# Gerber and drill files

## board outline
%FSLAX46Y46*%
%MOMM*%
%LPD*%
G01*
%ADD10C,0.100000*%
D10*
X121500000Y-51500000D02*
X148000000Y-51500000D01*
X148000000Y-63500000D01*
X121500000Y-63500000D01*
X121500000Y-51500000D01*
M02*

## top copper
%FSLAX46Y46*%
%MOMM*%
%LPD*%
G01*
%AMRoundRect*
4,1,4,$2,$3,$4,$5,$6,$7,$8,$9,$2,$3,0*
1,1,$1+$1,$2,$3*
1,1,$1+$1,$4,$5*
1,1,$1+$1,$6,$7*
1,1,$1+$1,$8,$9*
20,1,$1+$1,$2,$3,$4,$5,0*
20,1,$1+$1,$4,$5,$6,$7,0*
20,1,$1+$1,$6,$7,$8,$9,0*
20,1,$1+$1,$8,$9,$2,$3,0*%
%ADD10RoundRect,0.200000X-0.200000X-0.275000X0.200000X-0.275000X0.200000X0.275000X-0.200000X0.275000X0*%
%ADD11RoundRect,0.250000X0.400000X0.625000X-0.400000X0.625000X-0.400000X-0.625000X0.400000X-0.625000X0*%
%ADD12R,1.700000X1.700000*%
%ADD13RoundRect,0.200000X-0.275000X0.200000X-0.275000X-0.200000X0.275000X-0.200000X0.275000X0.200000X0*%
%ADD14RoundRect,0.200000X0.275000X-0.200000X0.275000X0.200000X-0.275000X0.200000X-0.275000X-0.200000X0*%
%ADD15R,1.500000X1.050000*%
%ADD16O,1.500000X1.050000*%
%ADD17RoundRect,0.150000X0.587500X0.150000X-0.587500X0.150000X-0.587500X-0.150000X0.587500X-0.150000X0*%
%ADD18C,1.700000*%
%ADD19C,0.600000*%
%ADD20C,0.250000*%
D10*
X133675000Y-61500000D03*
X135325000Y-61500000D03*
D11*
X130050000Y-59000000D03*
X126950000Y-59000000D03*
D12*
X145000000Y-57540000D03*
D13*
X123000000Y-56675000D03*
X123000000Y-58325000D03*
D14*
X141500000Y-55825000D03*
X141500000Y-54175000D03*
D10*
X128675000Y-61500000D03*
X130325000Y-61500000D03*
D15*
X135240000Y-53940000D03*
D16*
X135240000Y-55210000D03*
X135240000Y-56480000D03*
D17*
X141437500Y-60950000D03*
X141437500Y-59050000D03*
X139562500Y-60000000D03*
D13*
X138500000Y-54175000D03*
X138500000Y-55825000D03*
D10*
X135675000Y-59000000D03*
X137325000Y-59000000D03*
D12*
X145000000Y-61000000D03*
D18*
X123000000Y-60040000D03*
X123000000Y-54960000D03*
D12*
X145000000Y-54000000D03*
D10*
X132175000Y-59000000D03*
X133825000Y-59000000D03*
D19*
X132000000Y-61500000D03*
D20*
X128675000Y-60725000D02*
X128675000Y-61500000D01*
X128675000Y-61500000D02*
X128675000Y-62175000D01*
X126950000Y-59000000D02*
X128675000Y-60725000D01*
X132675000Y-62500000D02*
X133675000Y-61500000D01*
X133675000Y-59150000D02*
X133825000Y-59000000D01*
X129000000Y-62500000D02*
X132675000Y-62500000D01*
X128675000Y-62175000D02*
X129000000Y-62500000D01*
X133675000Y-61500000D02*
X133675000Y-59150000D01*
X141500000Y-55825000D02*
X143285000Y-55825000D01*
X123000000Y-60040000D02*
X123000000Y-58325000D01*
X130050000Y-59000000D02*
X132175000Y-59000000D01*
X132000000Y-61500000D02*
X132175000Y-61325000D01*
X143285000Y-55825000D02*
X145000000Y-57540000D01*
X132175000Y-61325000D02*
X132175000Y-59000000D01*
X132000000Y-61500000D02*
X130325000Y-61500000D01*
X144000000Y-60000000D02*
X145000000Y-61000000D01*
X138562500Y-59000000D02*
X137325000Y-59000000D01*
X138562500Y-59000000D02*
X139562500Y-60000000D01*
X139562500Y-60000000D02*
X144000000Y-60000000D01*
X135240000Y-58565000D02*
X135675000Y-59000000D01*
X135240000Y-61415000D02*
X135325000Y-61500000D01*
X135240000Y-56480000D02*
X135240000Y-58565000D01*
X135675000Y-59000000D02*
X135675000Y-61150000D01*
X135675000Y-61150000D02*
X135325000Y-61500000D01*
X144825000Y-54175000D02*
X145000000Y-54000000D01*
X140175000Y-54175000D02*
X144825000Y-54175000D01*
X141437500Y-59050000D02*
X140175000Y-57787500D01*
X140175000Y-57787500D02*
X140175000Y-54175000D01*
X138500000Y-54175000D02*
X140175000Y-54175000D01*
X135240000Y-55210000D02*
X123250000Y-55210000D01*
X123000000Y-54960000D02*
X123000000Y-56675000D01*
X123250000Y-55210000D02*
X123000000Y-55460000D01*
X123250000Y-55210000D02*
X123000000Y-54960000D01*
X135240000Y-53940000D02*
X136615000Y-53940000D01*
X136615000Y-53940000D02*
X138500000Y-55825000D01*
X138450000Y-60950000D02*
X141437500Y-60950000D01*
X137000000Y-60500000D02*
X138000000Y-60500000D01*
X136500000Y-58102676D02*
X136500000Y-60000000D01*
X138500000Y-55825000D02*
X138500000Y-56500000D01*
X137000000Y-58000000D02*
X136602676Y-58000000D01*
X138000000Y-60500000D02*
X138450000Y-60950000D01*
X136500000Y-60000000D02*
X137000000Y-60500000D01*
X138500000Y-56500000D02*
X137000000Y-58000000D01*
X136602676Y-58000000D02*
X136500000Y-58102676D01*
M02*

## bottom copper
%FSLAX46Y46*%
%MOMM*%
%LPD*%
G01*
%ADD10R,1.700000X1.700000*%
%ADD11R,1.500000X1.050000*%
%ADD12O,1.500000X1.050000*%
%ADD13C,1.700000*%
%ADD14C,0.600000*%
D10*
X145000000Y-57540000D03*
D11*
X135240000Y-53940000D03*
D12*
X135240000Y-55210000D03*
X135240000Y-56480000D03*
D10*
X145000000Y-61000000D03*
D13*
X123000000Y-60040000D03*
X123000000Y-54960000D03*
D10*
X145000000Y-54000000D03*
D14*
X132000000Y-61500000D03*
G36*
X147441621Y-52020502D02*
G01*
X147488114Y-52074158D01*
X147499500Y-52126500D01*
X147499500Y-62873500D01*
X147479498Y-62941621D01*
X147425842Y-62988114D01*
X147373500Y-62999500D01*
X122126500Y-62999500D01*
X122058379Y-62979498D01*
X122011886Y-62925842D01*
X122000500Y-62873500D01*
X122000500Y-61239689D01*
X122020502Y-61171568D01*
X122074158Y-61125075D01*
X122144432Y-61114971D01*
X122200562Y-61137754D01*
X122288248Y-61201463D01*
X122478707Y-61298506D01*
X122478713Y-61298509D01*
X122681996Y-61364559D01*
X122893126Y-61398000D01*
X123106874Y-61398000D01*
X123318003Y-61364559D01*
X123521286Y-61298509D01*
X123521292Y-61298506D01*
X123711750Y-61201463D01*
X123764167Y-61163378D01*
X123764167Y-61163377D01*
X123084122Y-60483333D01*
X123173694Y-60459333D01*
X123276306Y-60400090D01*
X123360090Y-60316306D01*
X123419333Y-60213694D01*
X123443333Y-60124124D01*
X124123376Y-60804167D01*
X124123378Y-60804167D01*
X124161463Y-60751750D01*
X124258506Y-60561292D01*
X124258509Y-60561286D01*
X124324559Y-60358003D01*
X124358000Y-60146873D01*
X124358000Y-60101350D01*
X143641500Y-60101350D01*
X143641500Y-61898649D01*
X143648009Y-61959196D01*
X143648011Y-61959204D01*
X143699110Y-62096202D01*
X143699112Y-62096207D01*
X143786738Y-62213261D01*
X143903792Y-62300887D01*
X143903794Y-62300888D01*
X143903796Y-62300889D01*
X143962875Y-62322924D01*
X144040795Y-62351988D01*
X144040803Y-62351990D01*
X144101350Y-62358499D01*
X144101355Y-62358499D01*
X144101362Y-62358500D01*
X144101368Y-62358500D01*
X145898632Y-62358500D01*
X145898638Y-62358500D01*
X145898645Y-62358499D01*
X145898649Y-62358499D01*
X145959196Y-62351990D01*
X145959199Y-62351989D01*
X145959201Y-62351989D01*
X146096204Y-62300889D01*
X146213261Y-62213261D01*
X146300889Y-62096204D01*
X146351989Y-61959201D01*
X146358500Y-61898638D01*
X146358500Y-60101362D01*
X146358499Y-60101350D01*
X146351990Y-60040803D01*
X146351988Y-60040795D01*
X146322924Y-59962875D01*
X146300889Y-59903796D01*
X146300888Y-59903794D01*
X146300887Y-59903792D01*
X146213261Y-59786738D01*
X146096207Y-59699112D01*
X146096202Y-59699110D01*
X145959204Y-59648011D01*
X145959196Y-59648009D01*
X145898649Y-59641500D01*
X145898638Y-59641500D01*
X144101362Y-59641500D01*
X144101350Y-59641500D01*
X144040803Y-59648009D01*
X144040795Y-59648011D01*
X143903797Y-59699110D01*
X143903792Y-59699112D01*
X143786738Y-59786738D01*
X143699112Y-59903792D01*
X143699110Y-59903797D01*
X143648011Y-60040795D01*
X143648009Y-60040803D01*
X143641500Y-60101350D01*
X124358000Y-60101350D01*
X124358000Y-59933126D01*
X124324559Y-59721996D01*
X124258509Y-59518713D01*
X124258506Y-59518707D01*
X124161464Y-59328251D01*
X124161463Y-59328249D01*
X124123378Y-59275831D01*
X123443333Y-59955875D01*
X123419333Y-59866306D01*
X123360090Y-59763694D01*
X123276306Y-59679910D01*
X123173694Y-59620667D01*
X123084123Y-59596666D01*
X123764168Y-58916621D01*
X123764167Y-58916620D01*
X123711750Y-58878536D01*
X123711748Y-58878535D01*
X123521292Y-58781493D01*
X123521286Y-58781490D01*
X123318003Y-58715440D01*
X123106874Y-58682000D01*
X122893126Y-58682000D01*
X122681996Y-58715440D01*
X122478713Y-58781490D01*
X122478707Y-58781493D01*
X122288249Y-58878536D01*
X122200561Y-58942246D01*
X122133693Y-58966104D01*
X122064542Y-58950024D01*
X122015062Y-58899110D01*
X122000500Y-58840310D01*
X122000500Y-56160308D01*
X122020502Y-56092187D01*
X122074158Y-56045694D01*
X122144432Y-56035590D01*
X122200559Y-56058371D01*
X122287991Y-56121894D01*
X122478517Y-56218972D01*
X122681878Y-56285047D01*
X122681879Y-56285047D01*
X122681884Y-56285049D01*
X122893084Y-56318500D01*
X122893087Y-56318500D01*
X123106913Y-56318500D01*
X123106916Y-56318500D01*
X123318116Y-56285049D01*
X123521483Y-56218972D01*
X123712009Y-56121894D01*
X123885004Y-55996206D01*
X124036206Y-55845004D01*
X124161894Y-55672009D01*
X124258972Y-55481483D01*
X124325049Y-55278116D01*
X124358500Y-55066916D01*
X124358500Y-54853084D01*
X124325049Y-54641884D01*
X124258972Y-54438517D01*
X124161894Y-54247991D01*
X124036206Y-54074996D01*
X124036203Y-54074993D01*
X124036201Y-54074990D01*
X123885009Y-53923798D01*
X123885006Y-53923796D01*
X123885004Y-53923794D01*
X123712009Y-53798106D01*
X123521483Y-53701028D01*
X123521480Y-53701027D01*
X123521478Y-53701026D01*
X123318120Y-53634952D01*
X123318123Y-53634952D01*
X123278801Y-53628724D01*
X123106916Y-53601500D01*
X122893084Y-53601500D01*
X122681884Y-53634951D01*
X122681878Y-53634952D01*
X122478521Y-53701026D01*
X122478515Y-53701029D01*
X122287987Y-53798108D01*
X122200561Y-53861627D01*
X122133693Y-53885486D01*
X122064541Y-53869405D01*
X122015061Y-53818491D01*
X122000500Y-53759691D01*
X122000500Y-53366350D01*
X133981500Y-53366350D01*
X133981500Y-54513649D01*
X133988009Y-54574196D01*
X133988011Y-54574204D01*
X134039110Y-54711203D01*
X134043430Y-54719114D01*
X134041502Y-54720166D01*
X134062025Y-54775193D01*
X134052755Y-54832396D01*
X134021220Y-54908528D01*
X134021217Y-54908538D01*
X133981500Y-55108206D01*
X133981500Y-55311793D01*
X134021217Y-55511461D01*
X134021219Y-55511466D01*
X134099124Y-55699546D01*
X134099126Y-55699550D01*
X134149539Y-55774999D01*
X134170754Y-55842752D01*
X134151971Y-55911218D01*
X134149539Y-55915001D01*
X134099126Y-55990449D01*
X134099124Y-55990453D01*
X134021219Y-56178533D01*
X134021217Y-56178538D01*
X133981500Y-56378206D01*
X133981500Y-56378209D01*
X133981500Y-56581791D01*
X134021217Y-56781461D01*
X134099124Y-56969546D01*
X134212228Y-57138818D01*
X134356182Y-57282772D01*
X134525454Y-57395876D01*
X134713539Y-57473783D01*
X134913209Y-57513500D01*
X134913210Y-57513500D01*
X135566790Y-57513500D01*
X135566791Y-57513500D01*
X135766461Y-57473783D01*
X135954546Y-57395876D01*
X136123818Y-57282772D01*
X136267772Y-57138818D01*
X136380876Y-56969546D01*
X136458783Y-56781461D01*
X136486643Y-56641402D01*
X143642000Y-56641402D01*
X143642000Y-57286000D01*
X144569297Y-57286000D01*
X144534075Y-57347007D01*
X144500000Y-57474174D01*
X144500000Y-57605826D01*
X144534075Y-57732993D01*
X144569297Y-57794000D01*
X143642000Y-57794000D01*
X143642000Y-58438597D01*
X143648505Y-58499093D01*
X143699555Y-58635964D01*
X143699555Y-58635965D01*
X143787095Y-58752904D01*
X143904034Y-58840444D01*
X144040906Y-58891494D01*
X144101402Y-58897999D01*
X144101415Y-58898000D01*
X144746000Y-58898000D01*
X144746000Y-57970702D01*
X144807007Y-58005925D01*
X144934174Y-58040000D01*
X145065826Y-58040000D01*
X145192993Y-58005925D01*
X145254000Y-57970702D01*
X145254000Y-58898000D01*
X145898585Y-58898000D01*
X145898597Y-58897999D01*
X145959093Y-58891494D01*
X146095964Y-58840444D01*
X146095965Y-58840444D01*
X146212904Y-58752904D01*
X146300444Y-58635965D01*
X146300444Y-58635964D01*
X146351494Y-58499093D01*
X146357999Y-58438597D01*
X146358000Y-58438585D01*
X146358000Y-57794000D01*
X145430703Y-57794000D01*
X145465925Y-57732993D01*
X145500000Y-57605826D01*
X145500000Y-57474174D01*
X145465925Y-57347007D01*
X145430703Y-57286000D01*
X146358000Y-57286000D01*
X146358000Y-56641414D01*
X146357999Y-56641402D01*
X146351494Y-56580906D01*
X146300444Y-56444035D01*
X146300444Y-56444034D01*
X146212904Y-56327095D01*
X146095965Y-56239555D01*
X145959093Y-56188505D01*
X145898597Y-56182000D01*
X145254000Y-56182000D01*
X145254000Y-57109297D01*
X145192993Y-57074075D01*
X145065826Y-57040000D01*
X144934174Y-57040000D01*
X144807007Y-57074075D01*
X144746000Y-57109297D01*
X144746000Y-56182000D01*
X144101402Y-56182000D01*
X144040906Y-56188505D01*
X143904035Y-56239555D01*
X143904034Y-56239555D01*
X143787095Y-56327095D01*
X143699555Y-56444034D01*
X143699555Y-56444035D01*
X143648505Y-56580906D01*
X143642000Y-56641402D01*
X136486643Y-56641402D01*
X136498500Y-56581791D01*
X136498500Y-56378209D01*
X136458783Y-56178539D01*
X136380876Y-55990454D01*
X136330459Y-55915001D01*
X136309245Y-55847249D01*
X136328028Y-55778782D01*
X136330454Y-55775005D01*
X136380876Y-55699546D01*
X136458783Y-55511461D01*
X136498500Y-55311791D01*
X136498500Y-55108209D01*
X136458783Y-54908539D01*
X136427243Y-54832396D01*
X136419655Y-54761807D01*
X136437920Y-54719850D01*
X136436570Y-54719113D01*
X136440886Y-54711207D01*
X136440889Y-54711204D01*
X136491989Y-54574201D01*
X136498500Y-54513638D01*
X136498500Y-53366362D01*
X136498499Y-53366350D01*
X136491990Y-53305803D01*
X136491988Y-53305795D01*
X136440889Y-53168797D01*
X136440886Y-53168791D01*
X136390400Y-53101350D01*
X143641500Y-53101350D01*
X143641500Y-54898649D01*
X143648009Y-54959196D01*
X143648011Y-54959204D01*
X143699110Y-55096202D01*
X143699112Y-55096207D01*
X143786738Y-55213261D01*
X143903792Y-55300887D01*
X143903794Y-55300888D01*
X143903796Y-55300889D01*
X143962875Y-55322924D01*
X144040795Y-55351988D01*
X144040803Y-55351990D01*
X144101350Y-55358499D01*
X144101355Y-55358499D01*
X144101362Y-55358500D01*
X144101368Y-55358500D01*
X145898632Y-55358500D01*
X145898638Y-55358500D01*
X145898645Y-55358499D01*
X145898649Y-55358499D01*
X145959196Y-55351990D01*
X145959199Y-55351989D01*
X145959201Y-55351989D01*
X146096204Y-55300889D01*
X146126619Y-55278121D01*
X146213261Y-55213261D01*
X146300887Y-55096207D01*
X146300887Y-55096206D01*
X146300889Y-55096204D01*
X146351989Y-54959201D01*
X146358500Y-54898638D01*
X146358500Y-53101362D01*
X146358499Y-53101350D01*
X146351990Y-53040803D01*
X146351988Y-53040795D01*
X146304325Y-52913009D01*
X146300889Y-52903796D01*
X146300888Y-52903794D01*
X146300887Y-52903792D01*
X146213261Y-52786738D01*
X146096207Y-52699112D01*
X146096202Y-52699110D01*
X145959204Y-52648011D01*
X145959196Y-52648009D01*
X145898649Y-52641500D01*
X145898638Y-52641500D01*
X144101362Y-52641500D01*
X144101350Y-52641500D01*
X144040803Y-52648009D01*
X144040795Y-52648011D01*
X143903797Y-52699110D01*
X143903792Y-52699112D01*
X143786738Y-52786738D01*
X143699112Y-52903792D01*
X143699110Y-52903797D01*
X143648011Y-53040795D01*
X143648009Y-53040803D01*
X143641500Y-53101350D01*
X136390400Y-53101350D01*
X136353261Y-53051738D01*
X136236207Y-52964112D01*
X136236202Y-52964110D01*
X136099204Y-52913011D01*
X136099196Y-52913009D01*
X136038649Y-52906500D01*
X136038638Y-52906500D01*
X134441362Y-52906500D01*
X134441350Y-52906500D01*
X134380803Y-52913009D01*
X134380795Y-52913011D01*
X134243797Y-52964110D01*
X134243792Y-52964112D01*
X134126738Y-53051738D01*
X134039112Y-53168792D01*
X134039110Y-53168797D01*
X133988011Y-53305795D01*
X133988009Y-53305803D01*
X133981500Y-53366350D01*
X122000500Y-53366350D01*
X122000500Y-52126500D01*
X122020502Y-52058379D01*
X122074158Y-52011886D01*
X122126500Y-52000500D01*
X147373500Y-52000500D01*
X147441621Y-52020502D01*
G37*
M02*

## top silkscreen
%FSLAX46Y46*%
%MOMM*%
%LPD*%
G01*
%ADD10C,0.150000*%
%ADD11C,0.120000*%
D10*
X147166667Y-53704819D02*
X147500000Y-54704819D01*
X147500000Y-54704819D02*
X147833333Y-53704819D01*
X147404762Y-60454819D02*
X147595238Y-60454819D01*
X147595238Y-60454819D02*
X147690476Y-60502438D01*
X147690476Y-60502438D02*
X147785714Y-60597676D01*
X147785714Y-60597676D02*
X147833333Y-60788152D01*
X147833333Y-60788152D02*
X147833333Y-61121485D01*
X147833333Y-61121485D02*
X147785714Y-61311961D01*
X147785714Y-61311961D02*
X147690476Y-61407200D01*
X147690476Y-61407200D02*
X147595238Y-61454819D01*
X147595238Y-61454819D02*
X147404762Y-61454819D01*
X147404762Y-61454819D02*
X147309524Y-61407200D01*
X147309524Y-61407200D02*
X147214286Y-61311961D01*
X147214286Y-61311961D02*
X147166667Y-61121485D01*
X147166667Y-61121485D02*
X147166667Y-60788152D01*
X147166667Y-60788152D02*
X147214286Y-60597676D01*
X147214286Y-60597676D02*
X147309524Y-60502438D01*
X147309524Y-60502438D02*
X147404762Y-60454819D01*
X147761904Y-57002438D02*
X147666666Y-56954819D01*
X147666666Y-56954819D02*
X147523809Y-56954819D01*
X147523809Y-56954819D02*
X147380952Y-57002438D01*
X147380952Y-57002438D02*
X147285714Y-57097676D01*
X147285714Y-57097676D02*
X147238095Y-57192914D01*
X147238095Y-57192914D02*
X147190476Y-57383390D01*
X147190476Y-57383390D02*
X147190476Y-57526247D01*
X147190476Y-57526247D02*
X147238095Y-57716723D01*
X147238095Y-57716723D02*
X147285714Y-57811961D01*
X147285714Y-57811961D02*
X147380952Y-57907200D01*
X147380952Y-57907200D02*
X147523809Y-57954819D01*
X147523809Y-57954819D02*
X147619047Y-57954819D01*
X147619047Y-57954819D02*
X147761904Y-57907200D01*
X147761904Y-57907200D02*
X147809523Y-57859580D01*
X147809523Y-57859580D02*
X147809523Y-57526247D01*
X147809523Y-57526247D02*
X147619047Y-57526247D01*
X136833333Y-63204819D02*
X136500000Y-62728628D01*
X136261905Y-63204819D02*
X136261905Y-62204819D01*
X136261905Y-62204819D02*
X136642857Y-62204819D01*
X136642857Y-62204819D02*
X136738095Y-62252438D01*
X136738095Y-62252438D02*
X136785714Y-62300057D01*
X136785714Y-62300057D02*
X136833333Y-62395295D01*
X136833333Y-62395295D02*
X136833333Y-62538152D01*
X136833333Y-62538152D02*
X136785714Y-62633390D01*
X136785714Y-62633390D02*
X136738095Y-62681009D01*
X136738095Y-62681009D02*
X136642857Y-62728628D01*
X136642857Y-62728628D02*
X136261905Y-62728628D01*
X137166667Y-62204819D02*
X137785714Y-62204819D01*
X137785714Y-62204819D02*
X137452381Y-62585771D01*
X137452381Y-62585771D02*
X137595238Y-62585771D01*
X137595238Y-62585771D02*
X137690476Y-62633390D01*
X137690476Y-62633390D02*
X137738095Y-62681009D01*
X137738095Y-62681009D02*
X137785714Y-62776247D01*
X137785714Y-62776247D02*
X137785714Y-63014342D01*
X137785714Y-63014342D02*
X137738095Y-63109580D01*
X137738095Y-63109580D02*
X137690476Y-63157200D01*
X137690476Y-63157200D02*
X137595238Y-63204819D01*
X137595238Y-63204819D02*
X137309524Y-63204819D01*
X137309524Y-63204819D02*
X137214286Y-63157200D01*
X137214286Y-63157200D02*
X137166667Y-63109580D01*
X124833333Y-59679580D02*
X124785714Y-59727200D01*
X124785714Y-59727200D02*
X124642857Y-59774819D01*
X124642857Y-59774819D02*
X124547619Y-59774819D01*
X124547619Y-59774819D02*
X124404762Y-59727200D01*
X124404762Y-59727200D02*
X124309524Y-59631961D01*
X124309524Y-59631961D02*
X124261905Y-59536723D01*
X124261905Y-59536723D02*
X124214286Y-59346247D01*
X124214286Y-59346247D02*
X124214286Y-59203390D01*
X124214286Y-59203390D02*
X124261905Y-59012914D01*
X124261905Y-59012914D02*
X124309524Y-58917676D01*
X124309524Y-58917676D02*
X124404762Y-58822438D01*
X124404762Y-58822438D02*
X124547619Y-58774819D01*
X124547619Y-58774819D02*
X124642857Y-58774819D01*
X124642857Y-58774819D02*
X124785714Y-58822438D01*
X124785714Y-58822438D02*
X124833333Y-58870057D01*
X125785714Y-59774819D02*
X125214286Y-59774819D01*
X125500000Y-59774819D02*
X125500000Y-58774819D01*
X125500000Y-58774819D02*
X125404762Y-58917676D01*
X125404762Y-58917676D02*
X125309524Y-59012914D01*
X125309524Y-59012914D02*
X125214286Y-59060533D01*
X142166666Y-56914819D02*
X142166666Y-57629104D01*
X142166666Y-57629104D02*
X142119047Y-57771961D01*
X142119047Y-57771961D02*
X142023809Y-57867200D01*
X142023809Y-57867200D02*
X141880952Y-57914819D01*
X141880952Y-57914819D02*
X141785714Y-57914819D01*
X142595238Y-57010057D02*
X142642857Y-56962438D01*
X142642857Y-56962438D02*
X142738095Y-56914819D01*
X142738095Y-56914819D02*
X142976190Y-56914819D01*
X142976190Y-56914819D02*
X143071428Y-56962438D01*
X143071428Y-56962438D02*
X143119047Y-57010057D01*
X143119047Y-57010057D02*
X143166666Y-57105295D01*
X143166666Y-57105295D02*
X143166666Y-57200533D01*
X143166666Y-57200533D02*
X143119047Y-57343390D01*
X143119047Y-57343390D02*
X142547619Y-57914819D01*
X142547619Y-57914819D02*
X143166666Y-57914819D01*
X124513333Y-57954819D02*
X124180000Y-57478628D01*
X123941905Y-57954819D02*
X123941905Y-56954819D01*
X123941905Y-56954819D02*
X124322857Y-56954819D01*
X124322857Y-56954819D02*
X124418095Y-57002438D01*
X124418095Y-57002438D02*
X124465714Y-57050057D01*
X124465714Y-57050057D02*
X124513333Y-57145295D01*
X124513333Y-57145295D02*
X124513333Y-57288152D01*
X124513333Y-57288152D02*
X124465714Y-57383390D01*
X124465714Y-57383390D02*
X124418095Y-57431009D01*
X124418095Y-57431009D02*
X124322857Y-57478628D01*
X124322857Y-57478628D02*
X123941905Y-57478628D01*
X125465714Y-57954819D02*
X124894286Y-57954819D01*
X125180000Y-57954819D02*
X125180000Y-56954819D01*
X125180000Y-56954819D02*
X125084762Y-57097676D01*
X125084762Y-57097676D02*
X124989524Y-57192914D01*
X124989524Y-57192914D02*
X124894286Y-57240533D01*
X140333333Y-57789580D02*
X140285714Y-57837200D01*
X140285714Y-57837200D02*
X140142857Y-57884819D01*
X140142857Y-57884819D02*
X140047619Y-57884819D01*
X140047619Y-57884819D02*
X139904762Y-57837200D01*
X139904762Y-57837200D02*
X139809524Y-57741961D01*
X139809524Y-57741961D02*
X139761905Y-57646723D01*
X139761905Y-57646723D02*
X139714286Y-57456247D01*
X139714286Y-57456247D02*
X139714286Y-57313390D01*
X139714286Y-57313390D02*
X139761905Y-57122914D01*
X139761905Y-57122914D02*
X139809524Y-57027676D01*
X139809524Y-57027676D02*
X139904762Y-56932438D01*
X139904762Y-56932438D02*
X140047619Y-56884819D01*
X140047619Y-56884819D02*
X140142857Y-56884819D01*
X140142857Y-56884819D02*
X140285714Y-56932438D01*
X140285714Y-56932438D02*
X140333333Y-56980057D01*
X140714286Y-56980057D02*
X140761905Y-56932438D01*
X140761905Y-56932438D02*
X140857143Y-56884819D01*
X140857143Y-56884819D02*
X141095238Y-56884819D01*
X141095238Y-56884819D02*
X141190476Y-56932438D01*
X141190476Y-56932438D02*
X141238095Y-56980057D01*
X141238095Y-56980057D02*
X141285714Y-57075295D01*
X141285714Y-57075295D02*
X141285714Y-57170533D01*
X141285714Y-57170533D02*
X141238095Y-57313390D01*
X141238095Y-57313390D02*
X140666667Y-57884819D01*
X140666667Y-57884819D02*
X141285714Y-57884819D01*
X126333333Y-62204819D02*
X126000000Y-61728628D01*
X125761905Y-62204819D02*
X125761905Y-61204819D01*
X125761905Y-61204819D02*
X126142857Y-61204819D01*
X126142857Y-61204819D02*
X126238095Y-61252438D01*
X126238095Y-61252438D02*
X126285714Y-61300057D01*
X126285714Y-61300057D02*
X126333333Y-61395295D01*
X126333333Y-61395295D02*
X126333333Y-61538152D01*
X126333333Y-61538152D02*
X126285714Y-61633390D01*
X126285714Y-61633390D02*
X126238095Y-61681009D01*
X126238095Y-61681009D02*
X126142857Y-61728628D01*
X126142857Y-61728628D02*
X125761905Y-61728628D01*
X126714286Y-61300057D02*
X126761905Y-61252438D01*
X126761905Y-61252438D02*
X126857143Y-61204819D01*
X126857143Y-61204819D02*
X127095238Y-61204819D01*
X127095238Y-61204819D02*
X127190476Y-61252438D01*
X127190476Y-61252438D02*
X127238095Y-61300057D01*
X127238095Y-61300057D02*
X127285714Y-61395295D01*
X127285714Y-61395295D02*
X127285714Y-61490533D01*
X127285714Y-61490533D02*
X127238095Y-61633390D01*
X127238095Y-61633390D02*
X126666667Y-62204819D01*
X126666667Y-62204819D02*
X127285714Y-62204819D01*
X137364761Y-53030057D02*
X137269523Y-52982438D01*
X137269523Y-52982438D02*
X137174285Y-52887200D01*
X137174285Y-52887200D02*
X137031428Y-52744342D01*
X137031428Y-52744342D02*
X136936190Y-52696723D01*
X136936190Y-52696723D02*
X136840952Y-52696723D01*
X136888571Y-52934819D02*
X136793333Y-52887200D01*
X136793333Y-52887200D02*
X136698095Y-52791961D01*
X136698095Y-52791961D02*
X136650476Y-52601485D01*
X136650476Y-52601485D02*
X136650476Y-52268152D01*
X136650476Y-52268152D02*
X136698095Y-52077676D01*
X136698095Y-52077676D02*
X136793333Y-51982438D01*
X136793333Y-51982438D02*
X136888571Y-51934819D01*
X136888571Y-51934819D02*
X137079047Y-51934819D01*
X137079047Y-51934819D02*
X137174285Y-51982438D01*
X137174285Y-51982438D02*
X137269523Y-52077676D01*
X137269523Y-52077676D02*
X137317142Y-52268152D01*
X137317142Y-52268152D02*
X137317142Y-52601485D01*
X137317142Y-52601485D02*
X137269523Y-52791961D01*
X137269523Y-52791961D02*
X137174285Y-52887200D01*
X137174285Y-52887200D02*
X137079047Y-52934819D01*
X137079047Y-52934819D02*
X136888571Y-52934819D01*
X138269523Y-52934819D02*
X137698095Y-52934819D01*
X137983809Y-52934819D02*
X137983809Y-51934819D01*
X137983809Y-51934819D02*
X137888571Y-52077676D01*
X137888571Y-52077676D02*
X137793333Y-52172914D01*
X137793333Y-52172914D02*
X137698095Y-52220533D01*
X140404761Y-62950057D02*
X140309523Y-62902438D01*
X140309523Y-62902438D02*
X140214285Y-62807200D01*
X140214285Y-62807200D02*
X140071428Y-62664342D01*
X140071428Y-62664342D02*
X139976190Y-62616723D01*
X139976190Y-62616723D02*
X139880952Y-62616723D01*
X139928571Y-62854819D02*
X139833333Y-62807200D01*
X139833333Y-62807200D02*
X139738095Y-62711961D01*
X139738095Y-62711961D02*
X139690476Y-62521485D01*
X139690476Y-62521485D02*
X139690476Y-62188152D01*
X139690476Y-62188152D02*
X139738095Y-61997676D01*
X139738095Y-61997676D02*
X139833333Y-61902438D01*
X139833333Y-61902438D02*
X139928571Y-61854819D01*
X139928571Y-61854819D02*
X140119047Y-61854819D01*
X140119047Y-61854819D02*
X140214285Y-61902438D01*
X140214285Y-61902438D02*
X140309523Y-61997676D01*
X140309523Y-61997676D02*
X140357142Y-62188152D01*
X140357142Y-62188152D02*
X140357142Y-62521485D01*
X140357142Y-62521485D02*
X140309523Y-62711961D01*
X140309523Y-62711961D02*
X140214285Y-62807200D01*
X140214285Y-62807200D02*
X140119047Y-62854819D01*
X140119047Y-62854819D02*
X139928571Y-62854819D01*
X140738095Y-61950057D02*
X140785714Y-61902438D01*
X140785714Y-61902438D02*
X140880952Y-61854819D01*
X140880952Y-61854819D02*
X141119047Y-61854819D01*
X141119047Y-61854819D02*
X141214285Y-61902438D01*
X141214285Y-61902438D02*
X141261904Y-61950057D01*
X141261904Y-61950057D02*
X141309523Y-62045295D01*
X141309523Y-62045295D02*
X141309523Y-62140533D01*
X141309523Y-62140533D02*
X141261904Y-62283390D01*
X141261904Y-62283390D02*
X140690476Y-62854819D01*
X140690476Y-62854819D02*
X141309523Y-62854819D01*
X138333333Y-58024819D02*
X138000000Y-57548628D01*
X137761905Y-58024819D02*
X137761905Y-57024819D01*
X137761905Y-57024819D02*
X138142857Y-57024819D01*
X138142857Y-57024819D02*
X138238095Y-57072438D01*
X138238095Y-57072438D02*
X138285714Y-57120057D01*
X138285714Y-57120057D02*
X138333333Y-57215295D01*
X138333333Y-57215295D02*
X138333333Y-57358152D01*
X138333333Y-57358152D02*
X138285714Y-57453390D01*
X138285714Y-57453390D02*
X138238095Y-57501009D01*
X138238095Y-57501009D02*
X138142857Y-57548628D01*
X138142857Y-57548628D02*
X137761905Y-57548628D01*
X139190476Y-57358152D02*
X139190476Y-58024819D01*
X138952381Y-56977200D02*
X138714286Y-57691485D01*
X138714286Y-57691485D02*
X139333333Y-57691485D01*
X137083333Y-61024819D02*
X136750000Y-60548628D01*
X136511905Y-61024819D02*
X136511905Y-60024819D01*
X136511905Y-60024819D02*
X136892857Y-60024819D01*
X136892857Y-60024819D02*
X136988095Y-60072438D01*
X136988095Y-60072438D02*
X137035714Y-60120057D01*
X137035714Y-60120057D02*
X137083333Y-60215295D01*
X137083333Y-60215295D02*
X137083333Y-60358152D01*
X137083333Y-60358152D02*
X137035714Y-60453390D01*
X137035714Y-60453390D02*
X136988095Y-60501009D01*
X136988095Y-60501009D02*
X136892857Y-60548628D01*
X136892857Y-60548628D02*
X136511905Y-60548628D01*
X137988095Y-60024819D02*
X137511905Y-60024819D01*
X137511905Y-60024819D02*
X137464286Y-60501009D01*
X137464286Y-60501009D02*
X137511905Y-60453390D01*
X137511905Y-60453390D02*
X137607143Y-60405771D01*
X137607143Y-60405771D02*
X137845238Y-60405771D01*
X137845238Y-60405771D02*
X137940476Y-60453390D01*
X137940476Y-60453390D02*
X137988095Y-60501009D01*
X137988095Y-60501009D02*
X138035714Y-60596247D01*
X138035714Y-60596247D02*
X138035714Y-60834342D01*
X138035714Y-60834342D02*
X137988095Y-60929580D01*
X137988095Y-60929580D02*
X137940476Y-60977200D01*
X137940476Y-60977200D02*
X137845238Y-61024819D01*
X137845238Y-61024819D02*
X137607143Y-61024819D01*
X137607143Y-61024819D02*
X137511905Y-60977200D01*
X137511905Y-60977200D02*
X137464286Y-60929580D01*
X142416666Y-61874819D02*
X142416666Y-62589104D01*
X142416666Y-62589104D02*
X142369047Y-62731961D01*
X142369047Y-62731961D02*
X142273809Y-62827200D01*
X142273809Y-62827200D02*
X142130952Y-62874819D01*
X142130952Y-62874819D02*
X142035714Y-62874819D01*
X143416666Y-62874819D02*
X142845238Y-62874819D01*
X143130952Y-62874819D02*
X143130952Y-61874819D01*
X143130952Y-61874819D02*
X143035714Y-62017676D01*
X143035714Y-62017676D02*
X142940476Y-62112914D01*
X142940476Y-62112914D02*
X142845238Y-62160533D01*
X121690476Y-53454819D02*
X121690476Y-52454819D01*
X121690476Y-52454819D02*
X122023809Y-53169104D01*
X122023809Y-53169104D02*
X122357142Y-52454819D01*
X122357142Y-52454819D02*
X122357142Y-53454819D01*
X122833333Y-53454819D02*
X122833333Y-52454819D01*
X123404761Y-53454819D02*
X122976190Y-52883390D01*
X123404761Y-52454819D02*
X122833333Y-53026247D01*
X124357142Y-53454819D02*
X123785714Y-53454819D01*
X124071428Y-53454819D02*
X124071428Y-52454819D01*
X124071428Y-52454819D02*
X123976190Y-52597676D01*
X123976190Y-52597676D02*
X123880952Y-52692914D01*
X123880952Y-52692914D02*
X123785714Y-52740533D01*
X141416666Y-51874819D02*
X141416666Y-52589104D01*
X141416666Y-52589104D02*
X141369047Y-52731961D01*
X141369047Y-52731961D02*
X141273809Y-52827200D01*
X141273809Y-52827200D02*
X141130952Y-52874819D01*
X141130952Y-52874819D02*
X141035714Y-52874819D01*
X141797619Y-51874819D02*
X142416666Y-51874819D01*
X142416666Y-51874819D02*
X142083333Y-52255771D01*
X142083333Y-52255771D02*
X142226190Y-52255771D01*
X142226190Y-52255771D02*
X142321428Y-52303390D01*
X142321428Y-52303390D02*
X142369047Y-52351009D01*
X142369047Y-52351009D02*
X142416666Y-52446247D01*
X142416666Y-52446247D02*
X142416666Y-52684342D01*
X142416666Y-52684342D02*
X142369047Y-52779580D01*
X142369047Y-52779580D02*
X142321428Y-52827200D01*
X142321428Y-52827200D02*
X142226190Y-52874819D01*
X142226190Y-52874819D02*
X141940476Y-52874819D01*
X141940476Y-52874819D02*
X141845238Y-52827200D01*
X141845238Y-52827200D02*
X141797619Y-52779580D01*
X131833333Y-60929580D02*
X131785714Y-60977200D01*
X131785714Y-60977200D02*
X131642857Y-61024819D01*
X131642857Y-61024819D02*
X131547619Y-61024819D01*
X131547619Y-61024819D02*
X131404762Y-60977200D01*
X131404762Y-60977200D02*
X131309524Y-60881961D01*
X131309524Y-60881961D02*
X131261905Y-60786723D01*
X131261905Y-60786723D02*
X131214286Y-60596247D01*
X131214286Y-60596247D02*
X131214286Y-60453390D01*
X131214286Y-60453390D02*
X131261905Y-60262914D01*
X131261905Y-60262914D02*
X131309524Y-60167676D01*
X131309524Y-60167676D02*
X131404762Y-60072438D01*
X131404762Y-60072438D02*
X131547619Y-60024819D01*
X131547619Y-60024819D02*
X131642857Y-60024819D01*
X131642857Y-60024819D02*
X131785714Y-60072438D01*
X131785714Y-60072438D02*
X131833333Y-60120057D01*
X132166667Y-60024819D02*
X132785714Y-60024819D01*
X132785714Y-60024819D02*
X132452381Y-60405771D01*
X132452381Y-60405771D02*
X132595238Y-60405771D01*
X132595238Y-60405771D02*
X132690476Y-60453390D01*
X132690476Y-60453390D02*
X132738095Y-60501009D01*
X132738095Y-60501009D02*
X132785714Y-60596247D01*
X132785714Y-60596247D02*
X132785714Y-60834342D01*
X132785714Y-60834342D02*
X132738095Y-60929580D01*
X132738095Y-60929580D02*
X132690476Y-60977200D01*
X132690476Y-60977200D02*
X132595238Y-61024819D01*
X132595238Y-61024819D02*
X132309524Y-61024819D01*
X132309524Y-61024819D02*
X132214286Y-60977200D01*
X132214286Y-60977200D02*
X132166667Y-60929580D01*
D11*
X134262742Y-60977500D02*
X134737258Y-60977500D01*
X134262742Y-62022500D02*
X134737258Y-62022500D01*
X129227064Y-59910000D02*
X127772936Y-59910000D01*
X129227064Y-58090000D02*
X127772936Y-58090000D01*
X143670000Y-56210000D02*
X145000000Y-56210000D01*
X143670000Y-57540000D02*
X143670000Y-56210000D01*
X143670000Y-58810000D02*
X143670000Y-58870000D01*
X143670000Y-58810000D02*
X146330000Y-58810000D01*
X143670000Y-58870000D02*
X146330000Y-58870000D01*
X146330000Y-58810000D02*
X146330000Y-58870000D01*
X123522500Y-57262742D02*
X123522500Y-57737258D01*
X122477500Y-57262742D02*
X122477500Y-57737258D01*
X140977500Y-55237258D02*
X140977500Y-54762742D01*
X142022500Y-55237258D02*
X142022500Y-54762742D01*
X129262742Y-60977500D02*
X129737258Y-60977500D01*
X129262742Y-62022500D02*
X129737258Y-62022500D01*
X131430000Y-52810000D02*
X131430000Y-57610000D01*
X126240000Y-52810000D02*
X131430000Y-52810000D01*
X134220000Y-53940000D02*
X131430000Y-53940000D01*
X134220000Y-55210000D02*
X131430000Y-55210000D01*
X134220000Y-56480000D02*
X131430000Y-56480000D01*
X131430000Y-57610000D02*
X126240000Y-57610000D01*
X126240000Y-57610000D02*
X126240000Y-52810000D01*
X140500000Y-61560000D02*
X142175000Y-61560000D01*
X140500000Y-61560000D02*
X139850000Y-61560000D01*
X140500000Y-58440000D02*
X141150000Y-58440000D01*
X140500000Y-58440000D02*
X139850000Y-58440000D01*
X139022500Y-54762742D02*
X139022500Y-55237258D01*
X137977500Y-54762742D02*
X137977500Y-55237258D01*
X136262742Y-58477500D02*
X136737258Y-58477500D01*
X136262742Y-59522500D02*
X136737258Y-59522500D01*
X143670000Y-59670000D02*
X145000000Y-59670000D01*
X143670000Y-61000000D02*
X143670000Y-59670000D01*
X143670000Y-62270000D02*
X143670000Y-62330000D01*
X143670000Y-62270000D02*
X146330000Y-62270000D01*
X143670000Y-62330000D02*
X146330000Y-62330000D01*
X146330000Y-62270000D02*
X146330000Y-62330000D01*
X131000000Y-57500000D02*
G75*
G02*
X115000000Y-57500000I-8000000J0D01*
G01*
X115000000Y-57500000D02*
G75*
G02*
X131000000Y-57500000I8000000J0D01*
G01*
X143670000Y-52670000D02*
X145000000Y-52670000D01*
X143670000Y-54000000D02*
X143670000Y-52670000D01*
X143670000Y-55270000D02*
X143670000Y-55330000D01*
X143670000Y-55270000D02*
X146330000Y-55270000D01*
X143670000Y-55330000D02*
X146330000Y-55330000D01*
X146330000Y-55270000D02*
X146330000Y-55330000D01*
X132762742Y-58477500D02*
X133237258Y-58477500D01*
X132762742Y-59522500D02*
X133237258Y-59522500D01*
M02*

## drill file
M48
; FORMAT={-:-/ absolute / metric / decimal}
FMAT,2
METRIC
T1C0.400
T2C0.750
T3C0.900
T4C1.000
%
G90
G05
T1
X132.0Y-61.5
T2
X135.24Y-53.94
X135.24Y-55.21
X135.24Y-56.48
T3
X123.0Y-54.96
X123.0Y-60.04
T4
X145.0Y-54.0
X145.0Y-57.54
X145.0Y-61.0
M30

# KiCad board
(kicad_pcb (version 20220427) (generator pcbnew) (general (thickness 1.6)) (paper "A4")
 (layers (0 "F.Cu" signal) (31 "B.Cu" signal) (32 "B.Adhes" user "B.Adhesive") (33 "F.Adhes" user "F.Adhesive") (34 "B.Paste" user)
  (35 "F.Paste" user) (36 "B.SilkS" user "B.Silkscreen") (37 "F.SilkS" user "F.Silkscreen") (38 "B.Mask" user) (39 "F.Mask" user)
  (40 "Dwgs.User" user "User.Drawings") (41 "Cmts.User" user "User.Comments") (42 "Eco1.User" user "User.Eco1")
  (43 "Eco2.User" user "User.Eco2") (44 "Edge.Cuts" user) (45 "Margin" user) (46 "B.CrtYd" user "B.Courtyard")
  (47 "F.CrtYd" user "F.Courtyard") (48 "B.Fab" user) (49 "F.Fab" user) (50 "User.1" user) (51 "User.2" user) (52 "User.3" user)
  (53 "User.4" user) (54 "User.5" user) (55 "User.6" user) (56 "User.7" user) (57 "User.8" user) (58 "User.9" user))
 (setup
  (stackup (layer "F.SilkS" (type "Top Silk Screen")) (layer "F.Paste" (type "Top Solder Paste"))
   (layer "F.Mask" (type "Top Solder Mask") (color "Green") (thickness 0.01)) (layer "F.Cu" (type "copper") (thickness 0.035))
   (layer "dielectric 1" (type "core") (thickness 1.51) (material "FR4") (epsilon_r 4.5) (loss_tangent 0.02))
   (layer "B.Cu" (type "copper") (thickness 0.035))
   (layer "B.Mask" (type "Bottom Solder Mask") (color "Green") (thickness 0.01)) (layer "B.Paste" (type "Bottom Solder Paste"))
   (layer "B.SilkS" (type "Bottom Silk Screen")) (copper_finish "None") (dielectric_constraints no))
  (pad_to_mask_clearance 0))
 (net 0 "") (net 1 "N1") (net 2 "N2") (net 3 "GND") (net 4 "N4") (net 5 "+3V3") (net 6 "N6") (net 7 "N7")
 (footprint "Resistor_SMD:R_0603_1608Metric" (layer "F.Cu") (at 134.5 61.5)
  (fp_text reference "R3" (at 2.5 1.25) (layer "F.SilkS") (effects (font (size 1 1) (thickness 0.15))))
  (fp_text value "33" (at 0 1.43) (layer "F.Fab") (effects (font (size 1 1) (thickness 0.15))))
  (fp_line (start -0.237258 -0.5225) (end 0.237258 -0.5225) (stroke (width 0.12) (type solid)) (layer "F.SilkS"))
  (fp_line (start -0.237258 0.5225) (end 0.237258 0.5225) (stroke (width 0.12) (type solid)) (layer "F.SilkS"))
  (pad "1" smd roundrect locked (at -0.825 0) (size 0.8 0.95) (layers "F.Cu" "F.Paste" "F.Mask") (roundrect_rratio 0.25) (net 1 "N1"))
  (pad "2" smd roundrect locked (at 0.825 0) (size 0.8 0.95) (layers "F.Cu" "F.Paste" "F.Mask") (roundrect_rratio 0.25) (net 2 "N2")))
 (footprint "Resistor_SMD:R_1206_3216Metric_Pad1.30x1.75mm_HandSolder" (layer "F.Cu") (at 128.5 59 180)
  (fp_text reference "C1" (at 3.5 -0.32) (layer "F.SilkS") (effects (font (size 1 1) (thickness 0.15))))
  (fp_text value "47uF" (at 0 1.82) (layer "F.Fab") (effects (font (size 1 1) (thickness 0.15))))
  (fp_line (start -0.727064 -0.91) (end 0.727064 -0.91) (stroke (width 0.12) (type solid)) (layer "F.SilkS"))
  (fp_line (start -0.727064 0.91) (end 0.727064 0.91) (stroke (width 0.12) (type solid)) (layer "F.SilkS"))
  (pad "1" smd roundrect locked (at -1.55 0 180) (size 1.3 1.75) (layers "F.Cu" "F.Paste" "F.Mask") (roundrect_rratio 0.1923076923)
   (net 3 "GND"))
  (pad "2" smd roundrect locked (at 1.55 0 180) (size 1.3 1.75) (layers "F.Cu" "F.Paste" "F.Mask") (roundrect_rratio 0.1923076923)
   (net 1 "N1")))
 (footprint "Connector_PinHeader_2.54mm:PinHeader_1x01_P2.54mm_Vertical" (layer "F.Cu") (at 145 57.54)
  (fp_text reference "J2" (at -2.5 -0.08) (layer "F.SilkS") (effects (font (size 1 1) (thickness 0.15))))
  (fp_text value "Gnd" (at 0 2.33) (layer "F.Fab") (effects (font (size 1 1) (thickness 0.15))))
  (fp_line (start -1.33 -1.33) (end 0 -1.33) (stroke (width 0.12) (type solid)) (layer "F.SilkS"))
  (fp_line (start -1.33 0) (end -1.33 -1.33) (stroke (width 0.12) (type solid)) (layer "F.SilkS"))
  (fp_line (start -1.33 1.27) (end -1.33 1.33) (stroke (width 0.12) (type solid)) (layer "F.SilkS"))
  (fp_line (start -1.33 1.27) (end 1.33 1.27) (stroke (width 0.12) (type solid)) (layer "F.SilkS"))
  (fp_line (start -1.33 1.33) (end 1.33 1.33) (stroke (width 0.12) (type solid)) (layer "F.SilkS"))
  (fp_line (start 1.33 1.27) (end 1.33 1.33) (stroke (width 0.12) (type solid)) (layer "F.SilkS"))
  (pad "1" thru_hole rect locked (at 0 0) (size 1.7 1.7) (drill 1) (layers *.Cu *.Mask) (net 3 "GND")))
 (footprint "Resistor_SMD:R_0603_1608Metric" (layer "F.Cu") (at 123 57.5 -90)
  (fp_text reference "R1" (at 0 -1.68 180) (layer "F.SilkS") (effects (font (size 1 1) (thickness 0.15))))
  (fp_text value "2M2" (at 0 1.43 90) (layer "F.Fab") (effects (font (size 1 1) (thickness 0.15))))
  (fp_line (start -0.237258 -0.5225) (end 0.237258 -0.5225) (stroke (width 0.12) (type solid)) (layer "F.SilkS"))
  (fp_line (start -0.237258 0.5225) (end 0.237258 0.5225) (stroke (width 0.12) (type solid)) (layer "F.SilkS"))
  (pad "1" smd roundrect locked (at -0.825 0 270) (size 0.8 0.95) (layers "F.Cu" "F.Paste" "F.Mask") (roundrect_rratio 0.25) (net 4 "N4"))
  (pad "2" smd roundrect locked (at 0.825 0 270) (size 0.8 0.95) (layers "F.Cu" "F.Paste" "F.Mask") (roundrect_rratio 0.25) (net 3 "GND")))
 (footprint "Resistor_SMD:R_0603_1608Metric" (layer "F.Cu") (at 141.5 55 90)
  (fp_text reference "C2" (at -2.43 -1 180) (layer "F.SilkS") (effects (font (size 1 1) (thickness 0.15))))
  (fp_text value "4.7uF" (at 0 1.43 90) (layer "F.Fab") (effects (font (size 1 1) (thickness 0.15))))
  (fp_line (start -0.237258 -0.5225) (end 0.237258 -0.5225) (stroke (width 0.12) (type solid)) (layer "F.SilkS"))
  (fp_line (start -0.237258 0.5225) (end 0.237258 0.5225) (stroke (width 0.12) (type solid)) (layer "F.SilkS"))
  (pad "1" smd roundrect locked (at -0.825 0 90) (size 0.8 0.95) (layers "F.Cu" "F.Paste" "F.Mask") (roundrect_rratio 0.25) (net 3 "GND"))
  (pad "2" smd roundrect locked (at 0.825 0 90) (size 0.8 0.95) (layers "F.Cu" "F.Paste" "F.Mask") (roundrect_rratio 0.25) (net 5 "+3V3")))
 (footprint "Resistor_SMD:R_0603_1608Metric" (layer "F.Cu") (at 129.5 61.5)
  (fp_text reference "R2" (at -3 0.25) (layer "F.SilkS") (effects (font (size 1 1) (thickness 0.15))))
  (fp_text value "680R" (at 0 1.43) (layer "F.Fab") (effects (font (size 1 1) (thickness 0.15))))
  (fp_line (start -0.237258 -0.5225) (end 0.237258 -0.5225) (stroke (width 0.12) (type solid)) (layer "F.SilkS"))
  (fp_line (start -0.237258 0.5225) (end 0.237258 0.5225) (stroke (width 0.12) (type solid)) (layer "F.SilkS"))
  (pad "1" smd roundrect locked (at -0.825 0) (size 0.8 0.95) (layers "F.Cu" "F.Paste" "F.Mask") (roundrect_rratio 0.25) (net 1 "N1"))
  (pad "2" smd roundrect locked (at 0.825 0) (size 0.8 0.95) (layers "F.Cu" "F.Paste" "F.Mask") (roundrect_rratio 0.25) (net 3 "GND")))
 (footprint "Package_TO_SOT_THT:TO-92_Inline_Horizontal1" (layer "F.Cu") (at 135.24 53.94 -90)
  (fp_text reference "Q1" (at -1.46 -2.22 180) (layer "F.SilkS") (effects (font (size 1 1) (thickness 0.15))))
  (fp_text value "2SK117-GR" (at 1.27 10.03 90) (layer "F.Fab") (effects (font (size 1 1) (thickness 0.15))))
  (fp_line (start -1.13 3.81) (end 3.67 3.81) (stroke (width 0.12) (type solid)) (layer "F.SilkS"))
  (fp_line (start -1.13 9) (end -1.13 3.81) (stroke (width 0.12) (type solid)) (layer "F.SilkS"))
  (fp_line (start 0 1.02) (end 0 3.81) (stroke (width 0.12) (type solid)) (layer "F.SilkS"))
  (fp_line (start 1.27 1.02) (end 1.27 3.81) (stroke (width 0.12) (type solid)) (layer "F.SilkS"))
  (fp_line (start 2.54 1.02) (end 2.54 3.81) (stroke (width 0.12) (type solid)) (layer "F.SilkS"))
  (fp_line (start 3.67 3.81) (end 3.67 9) (stroke (width 0.12) (type solid)) (layer "F.SilkS"))
  (fp_line (start 3.67 9) (end -1.13 9) (stroke (width 0.12) (type solid)) (layer "F.SilkS"))
  (pad "1" thru_hole rect locked (at 0 0 270) (size 1.05 1.5) (drill 0.75) (layers *.Cu *.Mask) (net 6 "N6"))
  (pad "2" thru_hole oval locked (at 1.27 0 270) (size 1.05 1.5) (drill 0.75) (layers *.Cu *.Mask) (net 4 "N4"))
  (pad "3" thru_hole oval locked (at 2.54 0 270) (size 1.05 1.5) (drill 0.75) (layers *.Cu *.Mask) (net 2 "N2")))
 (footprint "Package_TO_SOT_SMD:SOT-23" (layer "F.Cu") (at 140.5 60 180)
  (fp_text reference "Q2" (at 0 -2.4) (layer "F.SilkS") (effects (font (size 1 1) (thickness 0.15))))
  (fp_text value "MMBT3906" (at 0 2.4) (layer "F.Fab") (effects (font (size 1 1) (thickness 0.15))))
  (fp_line (start 0 -1.56) (end -1.675 -1.56) (stroke (width 0.12) (type solid)) (layer "F.SilkS"))
  (fp_line (start 0 -1.56) (end 0.65 -1.56) (stroke (width 0.12) (type solid)) (layer "F.SilkS"))
  (fp_line (start 0 1.56) (end -0.65 1.56) (stroke (width 0.12) (type solid)) (layer "F.SilkS"))
  (fp_line (start 0 1.56) (end 0.65 1.56) (stroke (width 0.12) (type solid)) (layer "F.SilkS"))
  (pad "1" smd roundrect locked (at -0.9375 -0.95 180) (size 1.475 0.6) (layers "F.Cu" "F.Paste" "F.Mask") (roundrect_rratio 0.25)
   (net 6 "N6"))
  (pad "2" smd roundrect locked (at -0.9375 0.95 180) (size 1.475 0.6) (layers "F.Cu" "F.Paste" "F.Mask") (roundrect_rratio 0.25)
   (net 5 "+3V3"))
  (pad "3" smd roundrect locked (at 0.9375 0 180) (size 1.475 0.6) (layers "F.Cu" "F.Paste" "F.Mask") (roundrect_rratio 0.25) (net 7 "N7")))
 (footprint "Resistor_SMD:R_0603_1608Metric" (layer "F.Cu") (at 138.5 55 -90)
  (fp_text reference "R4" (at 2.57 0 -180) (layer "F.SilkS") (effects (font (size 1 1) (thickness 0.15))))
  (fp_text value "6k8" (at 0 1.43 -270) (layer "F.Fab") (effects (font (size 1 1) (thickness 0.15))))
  (fp_line (start -0.237258 -0.5225) (end 0.237258 -0.5225) (stroke (width 0.12) (type solid)) (layer "F.SilkS"))
  (fp_line (start -0.237258 0.5225) (end 0.237258 0.5225) (stroke (width 0.12) (type solid)) (layer "F.SilkS"))
  (pad "1" smd roundrect locked (at -0.825 0 270) (size 0.8 0.95) (layers "F.Cu" "F.Paste" "F.Mask") (roundrect_rratio 0.25) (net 5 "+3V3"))
  (pad "2" smd roundrect locked (at 0.825 0 270) (size 0.8 0.95) (layers "F.Cu" "F.Paste" "F.Mask") (roundrect_rratio 0.25) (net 6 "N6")))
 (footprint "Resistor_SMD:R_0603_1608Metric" (layer "F.Cu") (at 136.5 59)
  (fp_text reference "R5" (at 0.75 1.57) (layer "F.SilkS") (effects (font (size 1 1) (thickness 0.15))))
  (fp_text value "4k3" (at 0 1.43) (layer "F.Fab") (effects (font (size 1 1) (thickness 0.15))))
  (fp_line (start -0.237258 -0.5225) (end 0.237258 -0.5225) (stroke (width 0.12) (type solid)) (layer "F.SilkS"))
  (fp_line (start -0.237258 0.5225) (end 0.237258 0.5225) (stroke (width 0.12) (type solid)) (layer "F.SilkS"))
  (pad "1" smd roundrect locked (at -0.825 0) (size 0.8 0.95) (layers "F.Cu" "F.Paste" "F.Mask") (roundrect_rratio 0.25) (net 2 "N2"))
  (pad "2" smd roundrect locked (at 0.825 0) (size 0.8 0.95) (layers "F.Cu" "F.Paste" "F.Mask") (roundrect_rratio 0.25) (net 7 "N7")))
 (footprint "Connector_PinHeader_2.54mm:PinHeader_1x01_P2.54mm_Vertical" (layer "F.Cu") (at 145 61)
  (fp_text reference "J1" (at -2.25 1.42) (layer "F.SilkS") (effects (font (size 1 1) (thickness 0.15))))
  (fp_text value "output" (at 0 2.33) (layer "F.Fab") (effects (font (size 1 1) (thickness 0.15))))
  (fp_line (start -1.33 -1.33) (end 0 -1.33) (stroke (width 0.12) (type solid)) (layer "F.SilkS"))
  (fp_line (start -1.33 0) (end -1.33 -1.33) (stroke (width 0.12) (type solid)) (layer "F.SilkS"))
  (fp_line (start -1.33 1.27) (end -1.33 1.33) (stroke (width 0.12) (type solid)) (layer "F.SilkS"))
  (fp_line (start -1.33 1.27) (end 1.33 1.27) (stroke (width 0.12) (type solid)) (layer "F.SilkS"))
  (fp_line (start -1.33 1.33) (end 1.33 1.33) (stroke (width 0.12) (type solid)) (layer "F.SilkS"))
  (fp_line (start 1.33 1.27) (end 1.33 1.33) (stroke (width 0.12) (type solid)) (layer "F.SilkS"))
  (pad "1" thru_hole rect locked (at 0 0) (size 1.7 1.7) (drill 1) (layers *.Cu *.Mask) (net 7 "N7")))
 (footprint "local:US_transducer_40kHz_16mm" (layer "F.Cu") (at 123 57.5 90)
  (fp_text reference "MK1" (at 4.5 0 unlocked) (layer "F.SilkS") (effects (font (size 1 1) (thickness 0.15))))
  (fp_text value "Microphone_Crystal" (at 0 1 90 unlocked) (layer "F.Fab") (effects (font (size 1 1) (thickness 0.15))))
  (fp_circle (center 0 0) (end 0 -8) (stroke (width 0.12) (type solid)) (fill none) (layer "F.SilkS"))
  (pad "1" thru_hole circle (at -2.54 0 90) (size 1.7 1.7) (drill 0.9) (layers *.Cu *.Mask) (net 3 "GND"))
  (pad "2" thru_hole circle (at 2.54 0 90) (size 1.7 1.7) (drill 0.9) (layers *.Cu *.Mask) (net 4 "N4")))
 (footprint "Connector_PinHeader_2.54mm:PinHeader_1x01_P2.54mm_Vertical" (layer "F.Cu") (at 145 54)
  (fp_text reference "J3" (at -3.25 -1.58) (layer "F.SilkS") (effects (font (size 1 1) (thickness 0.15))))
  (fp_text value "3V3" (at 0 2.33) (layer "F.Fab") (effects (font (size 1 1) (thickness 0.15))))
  (fp_line (start -1.33 -1.33) (end 0 -1.33) (stroke (width 0.12) (type solid)) (layer "F.SilkS"))
  (fp_line (start -1.33 0) (end -1.33 -1.33) (stroke (width 0.12) (type solid)) (layer "F.SilkS"))
  (fp_line (start -1.33 1.27) (end -1.33 1.33) (stroke (width 0.12) (type solid)) (layer "F.SilkS"))
  (fp_line (start -1.33 1.27) (end 1.33 1.27) (stroke (width 0.12) (type solid)) (layer "F.SilkS"))
  (fp_line (start -1.33 1.33) (end 1.33 1.33) (stroke (width 0.12) (type solid)) (layer "F.SilkS"))
  (fp_line (start 1.33 1.27) (end 1.33 1.33) (stroke (width 0.12) (type solid)) (layer "F.SilkS"))
  (pad "1" thru_hole rect locked (at 0 0) (size 1.7 1.7) (drill 1) (layers *.Cu *.Mask) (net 5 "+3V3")))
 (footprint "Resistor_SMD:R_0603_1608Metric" (layer "F.Cu") (at 133 59)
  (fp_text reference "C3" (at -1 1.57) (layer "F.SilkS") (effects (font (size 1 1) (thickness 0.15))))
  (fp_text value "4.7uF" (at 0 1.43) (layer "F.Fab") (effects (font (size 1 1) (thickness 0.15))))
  (fp_line (start -0.237258 -0.5225) (end 0.237258 -0.5225) (stroke (width 0.12) (type solid)) (layer "F.SilkS"))
  (fp_line (start -0.237258 0.5225) (end 0.237258 0.5225) (stroke (width 0.12) (type solid)) (layer "F.SilkS"))
  (pad "1" smd roundrect locked (at -0.825 0) (size 0.8 0.95) (layers "F.Cu" "F.Paste" "F.Mask") (roundrect_rratio 0.25) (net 3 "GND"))
  (pad "2" smd roundrect locked (at 0.825 0) (size 0.8 0.95) (layers "F.Cu" "F.Paste" "F.Mask") (roundrect_rratio 0.25) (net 1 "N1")))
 (gr_rect (start 121.5 51.5) (end 148 63.5) (stroke (width 0.1) (type solid)) (fill none) (layer "Edge.Cuts"))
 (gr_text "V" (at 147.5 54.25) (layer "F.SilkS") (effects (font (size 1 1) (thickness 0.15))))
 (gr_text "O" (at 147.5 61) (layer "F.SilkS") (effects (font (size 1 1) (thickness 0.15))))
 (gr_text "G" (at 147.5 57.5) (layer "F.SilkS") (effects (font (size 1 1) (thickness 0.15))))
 (segment (start 128.675 60.725) (end 128.675 61.5) (width 0.25) (layer "F.Cu") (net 1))
 (segment (start 128.675 61.5) (end 128.675 62.175) (width 0.25) (layer "F.Cu") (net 1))
 (segment (start 126.95 59) (end 128.675 60.725) (width 0.25) (layer "F.Cu") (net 1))
 (segment (start 132.675 62.5) (end 133.675 61.5) (width 0.25) (layer "F.Cu") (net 1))
 (segment (start 133.675 59.15) (end 133.825 59) (width 0.25) (layer "F.Cu") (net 1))
 (segment (start 129 62.5) (end 132.675 62.5) (width 0.25) (layer "F.Cu") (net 1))
 (segment (start 128.675 62.175) (end 129 62.5) (width 0.25) (layer "F.Cu") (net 1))
 (segment (start 133.675 61.5) (end 133.675 59.15) (width 0.25) (layer "F.Cu") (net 1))
 (segment (start 141.5 55.825) (end 143.285 55.825) (width 0.25) (layer "F.Cu") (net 3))
 (segment (start 123 60.04) (end 123 58.325) (width 0.25) (layer "F.Cu") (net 3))
 (segment (start 130.05 59) (end 132.175 59) (width 0.25) (layer "F.Cu") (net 3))
 (segment (start 132 61.5) (end 132.175 61.325) (width 0.25) (layer "F.Cu") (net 3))
 (segment (start 143.285 55.825) (end 145 57.54) (width 0.25) (layer "F.Cu") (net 3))
 (segment (start 132.175 61.325) (end 132.175 59) (width 0.25) (layer "F.Cu") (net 3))
 (segment (start 132 61.5) (end 130.325 61.5) (width 0.25) (layer "F.Cu") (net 3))
 (via (at 132 61.5) (size 0.6) (drill 0.4) (layers "F.Cu" "B.Cu") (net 3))
 (segment (start 144 60) (end 145 61) (width 0.25) (layer "F.Cu") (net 7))
 (segment (start 138.5625 59) (end 137.325 59) (width 0.25) (layer "F.Cu") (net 7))
 (segment (start 138.5625 59) (end 139.5625 60) (width 0.25) (layer "F.Cu") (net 7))
 (segment (start 139.5625 60) (end 144 60) (width 0.25) (layer "F.Cu") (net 7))
 (segment (start 135.24 58.565) (end 135.675 59) (width 0.25) (layer "F.Cu") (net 2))
 (segment (start 135.24 61.415) (end 135.325 61.5) (width 0.25) (layer "F.Cu") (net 2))
 (segment (start 135.24 56.48) (end 135.24 58.565) (width 0.25) (layer "F.Cu") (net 2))
 (segment (start 135.675 59) (end 135.675 61.15) (width 0.25) (layer "F.Cu") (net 2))
 (segment (start 135.675 61.15) (end 135.325 61.5) (width 0.25) (layer "F.Cu") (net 2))
 (segment (start 144.825 54.175) (end 145 54) (width 0.25) (layer "F.Cu") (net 5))
 (segment (start 140.175 54.175) (end 144.825 54.175) (width 0.25) (layer "F.Cu") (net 5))
 (segment (start 141.4375 59.05) (end 140.175 57.7875) (width 0.25) (layer "F.Cu") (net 5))
 (segment (start 140.175 57.7875) (end 140.175 54.175) (width 0.25) (layer "F.Cu") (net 5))
 (segment (start 138.5 54.175) (end 140.175 54.175) (width 0.25) (layer "F.Cu") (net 5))
 (segment (start 135.24 55.21) (end 123.25 55.21) (width 0.25) (layer "F.Cu") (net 4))
 (segment (start 123 54.96) (end 123 56.675) (width 0.25) (layer "F.Cu") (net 4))
 (segment (start 123.25 55.21) (end 123 55.46) (width 0.25) (layer "F.Cu") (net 4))
 (segment (start 123.25 55.21) (end 123 54.96) (width 0.25) (layer "F.Cu") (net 4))
 (segment (start 135.24 53.94) (end 136.615 53.94) (width 0.25) (layer "F.Cu") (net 6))
 (segment (start 136.615 53.94) (end 138.5 55.825) (width 0.25) (layer "F.Cu") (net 6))
 (segment (start 138.45 60.95) (end 141.4375 60.95) (width 0.25) (layer "F.Cu") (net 6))
 (segment (start 137 60.5) (end 138 60.5) (width 0.25) (layer "F.Cu") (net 6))
 (segment (start 136.5 58.102676) (end 136.5 60) (width 0.25) (layer "F.Cu") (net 6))
 (segment (start 138.5 55.825) (end 138.5 56.5) (width 0.25) (layer "F.Cu") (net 6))
 (segment (start 137 58) (end 136.602676 58) (width 0.25) (layer "F.Cu") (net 6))
 (segment (start 138 60.5) (end 138.45 60.95) (width 0.25) (layer "F.Cu") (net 6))
 (segment (start 136.5 60) (end 137 60.5) (width 0.25) (layer "F.Cu") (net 6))
 (segment (start 138.5 56.5) (end 137 58) (width 0.25) (layer "F.Cu") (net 6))
 (segment (start 136.602676 58) (end 136.5 58.102676) (width 0.25) (layer "F.Cu") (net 6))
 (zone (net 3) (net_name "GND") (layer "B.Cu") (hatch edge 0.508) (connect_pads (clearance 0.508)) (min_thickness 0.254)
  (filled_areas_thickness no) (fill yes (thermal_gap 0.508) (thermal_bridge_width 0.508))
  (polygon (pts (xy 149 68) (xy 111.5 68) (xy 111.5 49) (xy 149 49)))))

